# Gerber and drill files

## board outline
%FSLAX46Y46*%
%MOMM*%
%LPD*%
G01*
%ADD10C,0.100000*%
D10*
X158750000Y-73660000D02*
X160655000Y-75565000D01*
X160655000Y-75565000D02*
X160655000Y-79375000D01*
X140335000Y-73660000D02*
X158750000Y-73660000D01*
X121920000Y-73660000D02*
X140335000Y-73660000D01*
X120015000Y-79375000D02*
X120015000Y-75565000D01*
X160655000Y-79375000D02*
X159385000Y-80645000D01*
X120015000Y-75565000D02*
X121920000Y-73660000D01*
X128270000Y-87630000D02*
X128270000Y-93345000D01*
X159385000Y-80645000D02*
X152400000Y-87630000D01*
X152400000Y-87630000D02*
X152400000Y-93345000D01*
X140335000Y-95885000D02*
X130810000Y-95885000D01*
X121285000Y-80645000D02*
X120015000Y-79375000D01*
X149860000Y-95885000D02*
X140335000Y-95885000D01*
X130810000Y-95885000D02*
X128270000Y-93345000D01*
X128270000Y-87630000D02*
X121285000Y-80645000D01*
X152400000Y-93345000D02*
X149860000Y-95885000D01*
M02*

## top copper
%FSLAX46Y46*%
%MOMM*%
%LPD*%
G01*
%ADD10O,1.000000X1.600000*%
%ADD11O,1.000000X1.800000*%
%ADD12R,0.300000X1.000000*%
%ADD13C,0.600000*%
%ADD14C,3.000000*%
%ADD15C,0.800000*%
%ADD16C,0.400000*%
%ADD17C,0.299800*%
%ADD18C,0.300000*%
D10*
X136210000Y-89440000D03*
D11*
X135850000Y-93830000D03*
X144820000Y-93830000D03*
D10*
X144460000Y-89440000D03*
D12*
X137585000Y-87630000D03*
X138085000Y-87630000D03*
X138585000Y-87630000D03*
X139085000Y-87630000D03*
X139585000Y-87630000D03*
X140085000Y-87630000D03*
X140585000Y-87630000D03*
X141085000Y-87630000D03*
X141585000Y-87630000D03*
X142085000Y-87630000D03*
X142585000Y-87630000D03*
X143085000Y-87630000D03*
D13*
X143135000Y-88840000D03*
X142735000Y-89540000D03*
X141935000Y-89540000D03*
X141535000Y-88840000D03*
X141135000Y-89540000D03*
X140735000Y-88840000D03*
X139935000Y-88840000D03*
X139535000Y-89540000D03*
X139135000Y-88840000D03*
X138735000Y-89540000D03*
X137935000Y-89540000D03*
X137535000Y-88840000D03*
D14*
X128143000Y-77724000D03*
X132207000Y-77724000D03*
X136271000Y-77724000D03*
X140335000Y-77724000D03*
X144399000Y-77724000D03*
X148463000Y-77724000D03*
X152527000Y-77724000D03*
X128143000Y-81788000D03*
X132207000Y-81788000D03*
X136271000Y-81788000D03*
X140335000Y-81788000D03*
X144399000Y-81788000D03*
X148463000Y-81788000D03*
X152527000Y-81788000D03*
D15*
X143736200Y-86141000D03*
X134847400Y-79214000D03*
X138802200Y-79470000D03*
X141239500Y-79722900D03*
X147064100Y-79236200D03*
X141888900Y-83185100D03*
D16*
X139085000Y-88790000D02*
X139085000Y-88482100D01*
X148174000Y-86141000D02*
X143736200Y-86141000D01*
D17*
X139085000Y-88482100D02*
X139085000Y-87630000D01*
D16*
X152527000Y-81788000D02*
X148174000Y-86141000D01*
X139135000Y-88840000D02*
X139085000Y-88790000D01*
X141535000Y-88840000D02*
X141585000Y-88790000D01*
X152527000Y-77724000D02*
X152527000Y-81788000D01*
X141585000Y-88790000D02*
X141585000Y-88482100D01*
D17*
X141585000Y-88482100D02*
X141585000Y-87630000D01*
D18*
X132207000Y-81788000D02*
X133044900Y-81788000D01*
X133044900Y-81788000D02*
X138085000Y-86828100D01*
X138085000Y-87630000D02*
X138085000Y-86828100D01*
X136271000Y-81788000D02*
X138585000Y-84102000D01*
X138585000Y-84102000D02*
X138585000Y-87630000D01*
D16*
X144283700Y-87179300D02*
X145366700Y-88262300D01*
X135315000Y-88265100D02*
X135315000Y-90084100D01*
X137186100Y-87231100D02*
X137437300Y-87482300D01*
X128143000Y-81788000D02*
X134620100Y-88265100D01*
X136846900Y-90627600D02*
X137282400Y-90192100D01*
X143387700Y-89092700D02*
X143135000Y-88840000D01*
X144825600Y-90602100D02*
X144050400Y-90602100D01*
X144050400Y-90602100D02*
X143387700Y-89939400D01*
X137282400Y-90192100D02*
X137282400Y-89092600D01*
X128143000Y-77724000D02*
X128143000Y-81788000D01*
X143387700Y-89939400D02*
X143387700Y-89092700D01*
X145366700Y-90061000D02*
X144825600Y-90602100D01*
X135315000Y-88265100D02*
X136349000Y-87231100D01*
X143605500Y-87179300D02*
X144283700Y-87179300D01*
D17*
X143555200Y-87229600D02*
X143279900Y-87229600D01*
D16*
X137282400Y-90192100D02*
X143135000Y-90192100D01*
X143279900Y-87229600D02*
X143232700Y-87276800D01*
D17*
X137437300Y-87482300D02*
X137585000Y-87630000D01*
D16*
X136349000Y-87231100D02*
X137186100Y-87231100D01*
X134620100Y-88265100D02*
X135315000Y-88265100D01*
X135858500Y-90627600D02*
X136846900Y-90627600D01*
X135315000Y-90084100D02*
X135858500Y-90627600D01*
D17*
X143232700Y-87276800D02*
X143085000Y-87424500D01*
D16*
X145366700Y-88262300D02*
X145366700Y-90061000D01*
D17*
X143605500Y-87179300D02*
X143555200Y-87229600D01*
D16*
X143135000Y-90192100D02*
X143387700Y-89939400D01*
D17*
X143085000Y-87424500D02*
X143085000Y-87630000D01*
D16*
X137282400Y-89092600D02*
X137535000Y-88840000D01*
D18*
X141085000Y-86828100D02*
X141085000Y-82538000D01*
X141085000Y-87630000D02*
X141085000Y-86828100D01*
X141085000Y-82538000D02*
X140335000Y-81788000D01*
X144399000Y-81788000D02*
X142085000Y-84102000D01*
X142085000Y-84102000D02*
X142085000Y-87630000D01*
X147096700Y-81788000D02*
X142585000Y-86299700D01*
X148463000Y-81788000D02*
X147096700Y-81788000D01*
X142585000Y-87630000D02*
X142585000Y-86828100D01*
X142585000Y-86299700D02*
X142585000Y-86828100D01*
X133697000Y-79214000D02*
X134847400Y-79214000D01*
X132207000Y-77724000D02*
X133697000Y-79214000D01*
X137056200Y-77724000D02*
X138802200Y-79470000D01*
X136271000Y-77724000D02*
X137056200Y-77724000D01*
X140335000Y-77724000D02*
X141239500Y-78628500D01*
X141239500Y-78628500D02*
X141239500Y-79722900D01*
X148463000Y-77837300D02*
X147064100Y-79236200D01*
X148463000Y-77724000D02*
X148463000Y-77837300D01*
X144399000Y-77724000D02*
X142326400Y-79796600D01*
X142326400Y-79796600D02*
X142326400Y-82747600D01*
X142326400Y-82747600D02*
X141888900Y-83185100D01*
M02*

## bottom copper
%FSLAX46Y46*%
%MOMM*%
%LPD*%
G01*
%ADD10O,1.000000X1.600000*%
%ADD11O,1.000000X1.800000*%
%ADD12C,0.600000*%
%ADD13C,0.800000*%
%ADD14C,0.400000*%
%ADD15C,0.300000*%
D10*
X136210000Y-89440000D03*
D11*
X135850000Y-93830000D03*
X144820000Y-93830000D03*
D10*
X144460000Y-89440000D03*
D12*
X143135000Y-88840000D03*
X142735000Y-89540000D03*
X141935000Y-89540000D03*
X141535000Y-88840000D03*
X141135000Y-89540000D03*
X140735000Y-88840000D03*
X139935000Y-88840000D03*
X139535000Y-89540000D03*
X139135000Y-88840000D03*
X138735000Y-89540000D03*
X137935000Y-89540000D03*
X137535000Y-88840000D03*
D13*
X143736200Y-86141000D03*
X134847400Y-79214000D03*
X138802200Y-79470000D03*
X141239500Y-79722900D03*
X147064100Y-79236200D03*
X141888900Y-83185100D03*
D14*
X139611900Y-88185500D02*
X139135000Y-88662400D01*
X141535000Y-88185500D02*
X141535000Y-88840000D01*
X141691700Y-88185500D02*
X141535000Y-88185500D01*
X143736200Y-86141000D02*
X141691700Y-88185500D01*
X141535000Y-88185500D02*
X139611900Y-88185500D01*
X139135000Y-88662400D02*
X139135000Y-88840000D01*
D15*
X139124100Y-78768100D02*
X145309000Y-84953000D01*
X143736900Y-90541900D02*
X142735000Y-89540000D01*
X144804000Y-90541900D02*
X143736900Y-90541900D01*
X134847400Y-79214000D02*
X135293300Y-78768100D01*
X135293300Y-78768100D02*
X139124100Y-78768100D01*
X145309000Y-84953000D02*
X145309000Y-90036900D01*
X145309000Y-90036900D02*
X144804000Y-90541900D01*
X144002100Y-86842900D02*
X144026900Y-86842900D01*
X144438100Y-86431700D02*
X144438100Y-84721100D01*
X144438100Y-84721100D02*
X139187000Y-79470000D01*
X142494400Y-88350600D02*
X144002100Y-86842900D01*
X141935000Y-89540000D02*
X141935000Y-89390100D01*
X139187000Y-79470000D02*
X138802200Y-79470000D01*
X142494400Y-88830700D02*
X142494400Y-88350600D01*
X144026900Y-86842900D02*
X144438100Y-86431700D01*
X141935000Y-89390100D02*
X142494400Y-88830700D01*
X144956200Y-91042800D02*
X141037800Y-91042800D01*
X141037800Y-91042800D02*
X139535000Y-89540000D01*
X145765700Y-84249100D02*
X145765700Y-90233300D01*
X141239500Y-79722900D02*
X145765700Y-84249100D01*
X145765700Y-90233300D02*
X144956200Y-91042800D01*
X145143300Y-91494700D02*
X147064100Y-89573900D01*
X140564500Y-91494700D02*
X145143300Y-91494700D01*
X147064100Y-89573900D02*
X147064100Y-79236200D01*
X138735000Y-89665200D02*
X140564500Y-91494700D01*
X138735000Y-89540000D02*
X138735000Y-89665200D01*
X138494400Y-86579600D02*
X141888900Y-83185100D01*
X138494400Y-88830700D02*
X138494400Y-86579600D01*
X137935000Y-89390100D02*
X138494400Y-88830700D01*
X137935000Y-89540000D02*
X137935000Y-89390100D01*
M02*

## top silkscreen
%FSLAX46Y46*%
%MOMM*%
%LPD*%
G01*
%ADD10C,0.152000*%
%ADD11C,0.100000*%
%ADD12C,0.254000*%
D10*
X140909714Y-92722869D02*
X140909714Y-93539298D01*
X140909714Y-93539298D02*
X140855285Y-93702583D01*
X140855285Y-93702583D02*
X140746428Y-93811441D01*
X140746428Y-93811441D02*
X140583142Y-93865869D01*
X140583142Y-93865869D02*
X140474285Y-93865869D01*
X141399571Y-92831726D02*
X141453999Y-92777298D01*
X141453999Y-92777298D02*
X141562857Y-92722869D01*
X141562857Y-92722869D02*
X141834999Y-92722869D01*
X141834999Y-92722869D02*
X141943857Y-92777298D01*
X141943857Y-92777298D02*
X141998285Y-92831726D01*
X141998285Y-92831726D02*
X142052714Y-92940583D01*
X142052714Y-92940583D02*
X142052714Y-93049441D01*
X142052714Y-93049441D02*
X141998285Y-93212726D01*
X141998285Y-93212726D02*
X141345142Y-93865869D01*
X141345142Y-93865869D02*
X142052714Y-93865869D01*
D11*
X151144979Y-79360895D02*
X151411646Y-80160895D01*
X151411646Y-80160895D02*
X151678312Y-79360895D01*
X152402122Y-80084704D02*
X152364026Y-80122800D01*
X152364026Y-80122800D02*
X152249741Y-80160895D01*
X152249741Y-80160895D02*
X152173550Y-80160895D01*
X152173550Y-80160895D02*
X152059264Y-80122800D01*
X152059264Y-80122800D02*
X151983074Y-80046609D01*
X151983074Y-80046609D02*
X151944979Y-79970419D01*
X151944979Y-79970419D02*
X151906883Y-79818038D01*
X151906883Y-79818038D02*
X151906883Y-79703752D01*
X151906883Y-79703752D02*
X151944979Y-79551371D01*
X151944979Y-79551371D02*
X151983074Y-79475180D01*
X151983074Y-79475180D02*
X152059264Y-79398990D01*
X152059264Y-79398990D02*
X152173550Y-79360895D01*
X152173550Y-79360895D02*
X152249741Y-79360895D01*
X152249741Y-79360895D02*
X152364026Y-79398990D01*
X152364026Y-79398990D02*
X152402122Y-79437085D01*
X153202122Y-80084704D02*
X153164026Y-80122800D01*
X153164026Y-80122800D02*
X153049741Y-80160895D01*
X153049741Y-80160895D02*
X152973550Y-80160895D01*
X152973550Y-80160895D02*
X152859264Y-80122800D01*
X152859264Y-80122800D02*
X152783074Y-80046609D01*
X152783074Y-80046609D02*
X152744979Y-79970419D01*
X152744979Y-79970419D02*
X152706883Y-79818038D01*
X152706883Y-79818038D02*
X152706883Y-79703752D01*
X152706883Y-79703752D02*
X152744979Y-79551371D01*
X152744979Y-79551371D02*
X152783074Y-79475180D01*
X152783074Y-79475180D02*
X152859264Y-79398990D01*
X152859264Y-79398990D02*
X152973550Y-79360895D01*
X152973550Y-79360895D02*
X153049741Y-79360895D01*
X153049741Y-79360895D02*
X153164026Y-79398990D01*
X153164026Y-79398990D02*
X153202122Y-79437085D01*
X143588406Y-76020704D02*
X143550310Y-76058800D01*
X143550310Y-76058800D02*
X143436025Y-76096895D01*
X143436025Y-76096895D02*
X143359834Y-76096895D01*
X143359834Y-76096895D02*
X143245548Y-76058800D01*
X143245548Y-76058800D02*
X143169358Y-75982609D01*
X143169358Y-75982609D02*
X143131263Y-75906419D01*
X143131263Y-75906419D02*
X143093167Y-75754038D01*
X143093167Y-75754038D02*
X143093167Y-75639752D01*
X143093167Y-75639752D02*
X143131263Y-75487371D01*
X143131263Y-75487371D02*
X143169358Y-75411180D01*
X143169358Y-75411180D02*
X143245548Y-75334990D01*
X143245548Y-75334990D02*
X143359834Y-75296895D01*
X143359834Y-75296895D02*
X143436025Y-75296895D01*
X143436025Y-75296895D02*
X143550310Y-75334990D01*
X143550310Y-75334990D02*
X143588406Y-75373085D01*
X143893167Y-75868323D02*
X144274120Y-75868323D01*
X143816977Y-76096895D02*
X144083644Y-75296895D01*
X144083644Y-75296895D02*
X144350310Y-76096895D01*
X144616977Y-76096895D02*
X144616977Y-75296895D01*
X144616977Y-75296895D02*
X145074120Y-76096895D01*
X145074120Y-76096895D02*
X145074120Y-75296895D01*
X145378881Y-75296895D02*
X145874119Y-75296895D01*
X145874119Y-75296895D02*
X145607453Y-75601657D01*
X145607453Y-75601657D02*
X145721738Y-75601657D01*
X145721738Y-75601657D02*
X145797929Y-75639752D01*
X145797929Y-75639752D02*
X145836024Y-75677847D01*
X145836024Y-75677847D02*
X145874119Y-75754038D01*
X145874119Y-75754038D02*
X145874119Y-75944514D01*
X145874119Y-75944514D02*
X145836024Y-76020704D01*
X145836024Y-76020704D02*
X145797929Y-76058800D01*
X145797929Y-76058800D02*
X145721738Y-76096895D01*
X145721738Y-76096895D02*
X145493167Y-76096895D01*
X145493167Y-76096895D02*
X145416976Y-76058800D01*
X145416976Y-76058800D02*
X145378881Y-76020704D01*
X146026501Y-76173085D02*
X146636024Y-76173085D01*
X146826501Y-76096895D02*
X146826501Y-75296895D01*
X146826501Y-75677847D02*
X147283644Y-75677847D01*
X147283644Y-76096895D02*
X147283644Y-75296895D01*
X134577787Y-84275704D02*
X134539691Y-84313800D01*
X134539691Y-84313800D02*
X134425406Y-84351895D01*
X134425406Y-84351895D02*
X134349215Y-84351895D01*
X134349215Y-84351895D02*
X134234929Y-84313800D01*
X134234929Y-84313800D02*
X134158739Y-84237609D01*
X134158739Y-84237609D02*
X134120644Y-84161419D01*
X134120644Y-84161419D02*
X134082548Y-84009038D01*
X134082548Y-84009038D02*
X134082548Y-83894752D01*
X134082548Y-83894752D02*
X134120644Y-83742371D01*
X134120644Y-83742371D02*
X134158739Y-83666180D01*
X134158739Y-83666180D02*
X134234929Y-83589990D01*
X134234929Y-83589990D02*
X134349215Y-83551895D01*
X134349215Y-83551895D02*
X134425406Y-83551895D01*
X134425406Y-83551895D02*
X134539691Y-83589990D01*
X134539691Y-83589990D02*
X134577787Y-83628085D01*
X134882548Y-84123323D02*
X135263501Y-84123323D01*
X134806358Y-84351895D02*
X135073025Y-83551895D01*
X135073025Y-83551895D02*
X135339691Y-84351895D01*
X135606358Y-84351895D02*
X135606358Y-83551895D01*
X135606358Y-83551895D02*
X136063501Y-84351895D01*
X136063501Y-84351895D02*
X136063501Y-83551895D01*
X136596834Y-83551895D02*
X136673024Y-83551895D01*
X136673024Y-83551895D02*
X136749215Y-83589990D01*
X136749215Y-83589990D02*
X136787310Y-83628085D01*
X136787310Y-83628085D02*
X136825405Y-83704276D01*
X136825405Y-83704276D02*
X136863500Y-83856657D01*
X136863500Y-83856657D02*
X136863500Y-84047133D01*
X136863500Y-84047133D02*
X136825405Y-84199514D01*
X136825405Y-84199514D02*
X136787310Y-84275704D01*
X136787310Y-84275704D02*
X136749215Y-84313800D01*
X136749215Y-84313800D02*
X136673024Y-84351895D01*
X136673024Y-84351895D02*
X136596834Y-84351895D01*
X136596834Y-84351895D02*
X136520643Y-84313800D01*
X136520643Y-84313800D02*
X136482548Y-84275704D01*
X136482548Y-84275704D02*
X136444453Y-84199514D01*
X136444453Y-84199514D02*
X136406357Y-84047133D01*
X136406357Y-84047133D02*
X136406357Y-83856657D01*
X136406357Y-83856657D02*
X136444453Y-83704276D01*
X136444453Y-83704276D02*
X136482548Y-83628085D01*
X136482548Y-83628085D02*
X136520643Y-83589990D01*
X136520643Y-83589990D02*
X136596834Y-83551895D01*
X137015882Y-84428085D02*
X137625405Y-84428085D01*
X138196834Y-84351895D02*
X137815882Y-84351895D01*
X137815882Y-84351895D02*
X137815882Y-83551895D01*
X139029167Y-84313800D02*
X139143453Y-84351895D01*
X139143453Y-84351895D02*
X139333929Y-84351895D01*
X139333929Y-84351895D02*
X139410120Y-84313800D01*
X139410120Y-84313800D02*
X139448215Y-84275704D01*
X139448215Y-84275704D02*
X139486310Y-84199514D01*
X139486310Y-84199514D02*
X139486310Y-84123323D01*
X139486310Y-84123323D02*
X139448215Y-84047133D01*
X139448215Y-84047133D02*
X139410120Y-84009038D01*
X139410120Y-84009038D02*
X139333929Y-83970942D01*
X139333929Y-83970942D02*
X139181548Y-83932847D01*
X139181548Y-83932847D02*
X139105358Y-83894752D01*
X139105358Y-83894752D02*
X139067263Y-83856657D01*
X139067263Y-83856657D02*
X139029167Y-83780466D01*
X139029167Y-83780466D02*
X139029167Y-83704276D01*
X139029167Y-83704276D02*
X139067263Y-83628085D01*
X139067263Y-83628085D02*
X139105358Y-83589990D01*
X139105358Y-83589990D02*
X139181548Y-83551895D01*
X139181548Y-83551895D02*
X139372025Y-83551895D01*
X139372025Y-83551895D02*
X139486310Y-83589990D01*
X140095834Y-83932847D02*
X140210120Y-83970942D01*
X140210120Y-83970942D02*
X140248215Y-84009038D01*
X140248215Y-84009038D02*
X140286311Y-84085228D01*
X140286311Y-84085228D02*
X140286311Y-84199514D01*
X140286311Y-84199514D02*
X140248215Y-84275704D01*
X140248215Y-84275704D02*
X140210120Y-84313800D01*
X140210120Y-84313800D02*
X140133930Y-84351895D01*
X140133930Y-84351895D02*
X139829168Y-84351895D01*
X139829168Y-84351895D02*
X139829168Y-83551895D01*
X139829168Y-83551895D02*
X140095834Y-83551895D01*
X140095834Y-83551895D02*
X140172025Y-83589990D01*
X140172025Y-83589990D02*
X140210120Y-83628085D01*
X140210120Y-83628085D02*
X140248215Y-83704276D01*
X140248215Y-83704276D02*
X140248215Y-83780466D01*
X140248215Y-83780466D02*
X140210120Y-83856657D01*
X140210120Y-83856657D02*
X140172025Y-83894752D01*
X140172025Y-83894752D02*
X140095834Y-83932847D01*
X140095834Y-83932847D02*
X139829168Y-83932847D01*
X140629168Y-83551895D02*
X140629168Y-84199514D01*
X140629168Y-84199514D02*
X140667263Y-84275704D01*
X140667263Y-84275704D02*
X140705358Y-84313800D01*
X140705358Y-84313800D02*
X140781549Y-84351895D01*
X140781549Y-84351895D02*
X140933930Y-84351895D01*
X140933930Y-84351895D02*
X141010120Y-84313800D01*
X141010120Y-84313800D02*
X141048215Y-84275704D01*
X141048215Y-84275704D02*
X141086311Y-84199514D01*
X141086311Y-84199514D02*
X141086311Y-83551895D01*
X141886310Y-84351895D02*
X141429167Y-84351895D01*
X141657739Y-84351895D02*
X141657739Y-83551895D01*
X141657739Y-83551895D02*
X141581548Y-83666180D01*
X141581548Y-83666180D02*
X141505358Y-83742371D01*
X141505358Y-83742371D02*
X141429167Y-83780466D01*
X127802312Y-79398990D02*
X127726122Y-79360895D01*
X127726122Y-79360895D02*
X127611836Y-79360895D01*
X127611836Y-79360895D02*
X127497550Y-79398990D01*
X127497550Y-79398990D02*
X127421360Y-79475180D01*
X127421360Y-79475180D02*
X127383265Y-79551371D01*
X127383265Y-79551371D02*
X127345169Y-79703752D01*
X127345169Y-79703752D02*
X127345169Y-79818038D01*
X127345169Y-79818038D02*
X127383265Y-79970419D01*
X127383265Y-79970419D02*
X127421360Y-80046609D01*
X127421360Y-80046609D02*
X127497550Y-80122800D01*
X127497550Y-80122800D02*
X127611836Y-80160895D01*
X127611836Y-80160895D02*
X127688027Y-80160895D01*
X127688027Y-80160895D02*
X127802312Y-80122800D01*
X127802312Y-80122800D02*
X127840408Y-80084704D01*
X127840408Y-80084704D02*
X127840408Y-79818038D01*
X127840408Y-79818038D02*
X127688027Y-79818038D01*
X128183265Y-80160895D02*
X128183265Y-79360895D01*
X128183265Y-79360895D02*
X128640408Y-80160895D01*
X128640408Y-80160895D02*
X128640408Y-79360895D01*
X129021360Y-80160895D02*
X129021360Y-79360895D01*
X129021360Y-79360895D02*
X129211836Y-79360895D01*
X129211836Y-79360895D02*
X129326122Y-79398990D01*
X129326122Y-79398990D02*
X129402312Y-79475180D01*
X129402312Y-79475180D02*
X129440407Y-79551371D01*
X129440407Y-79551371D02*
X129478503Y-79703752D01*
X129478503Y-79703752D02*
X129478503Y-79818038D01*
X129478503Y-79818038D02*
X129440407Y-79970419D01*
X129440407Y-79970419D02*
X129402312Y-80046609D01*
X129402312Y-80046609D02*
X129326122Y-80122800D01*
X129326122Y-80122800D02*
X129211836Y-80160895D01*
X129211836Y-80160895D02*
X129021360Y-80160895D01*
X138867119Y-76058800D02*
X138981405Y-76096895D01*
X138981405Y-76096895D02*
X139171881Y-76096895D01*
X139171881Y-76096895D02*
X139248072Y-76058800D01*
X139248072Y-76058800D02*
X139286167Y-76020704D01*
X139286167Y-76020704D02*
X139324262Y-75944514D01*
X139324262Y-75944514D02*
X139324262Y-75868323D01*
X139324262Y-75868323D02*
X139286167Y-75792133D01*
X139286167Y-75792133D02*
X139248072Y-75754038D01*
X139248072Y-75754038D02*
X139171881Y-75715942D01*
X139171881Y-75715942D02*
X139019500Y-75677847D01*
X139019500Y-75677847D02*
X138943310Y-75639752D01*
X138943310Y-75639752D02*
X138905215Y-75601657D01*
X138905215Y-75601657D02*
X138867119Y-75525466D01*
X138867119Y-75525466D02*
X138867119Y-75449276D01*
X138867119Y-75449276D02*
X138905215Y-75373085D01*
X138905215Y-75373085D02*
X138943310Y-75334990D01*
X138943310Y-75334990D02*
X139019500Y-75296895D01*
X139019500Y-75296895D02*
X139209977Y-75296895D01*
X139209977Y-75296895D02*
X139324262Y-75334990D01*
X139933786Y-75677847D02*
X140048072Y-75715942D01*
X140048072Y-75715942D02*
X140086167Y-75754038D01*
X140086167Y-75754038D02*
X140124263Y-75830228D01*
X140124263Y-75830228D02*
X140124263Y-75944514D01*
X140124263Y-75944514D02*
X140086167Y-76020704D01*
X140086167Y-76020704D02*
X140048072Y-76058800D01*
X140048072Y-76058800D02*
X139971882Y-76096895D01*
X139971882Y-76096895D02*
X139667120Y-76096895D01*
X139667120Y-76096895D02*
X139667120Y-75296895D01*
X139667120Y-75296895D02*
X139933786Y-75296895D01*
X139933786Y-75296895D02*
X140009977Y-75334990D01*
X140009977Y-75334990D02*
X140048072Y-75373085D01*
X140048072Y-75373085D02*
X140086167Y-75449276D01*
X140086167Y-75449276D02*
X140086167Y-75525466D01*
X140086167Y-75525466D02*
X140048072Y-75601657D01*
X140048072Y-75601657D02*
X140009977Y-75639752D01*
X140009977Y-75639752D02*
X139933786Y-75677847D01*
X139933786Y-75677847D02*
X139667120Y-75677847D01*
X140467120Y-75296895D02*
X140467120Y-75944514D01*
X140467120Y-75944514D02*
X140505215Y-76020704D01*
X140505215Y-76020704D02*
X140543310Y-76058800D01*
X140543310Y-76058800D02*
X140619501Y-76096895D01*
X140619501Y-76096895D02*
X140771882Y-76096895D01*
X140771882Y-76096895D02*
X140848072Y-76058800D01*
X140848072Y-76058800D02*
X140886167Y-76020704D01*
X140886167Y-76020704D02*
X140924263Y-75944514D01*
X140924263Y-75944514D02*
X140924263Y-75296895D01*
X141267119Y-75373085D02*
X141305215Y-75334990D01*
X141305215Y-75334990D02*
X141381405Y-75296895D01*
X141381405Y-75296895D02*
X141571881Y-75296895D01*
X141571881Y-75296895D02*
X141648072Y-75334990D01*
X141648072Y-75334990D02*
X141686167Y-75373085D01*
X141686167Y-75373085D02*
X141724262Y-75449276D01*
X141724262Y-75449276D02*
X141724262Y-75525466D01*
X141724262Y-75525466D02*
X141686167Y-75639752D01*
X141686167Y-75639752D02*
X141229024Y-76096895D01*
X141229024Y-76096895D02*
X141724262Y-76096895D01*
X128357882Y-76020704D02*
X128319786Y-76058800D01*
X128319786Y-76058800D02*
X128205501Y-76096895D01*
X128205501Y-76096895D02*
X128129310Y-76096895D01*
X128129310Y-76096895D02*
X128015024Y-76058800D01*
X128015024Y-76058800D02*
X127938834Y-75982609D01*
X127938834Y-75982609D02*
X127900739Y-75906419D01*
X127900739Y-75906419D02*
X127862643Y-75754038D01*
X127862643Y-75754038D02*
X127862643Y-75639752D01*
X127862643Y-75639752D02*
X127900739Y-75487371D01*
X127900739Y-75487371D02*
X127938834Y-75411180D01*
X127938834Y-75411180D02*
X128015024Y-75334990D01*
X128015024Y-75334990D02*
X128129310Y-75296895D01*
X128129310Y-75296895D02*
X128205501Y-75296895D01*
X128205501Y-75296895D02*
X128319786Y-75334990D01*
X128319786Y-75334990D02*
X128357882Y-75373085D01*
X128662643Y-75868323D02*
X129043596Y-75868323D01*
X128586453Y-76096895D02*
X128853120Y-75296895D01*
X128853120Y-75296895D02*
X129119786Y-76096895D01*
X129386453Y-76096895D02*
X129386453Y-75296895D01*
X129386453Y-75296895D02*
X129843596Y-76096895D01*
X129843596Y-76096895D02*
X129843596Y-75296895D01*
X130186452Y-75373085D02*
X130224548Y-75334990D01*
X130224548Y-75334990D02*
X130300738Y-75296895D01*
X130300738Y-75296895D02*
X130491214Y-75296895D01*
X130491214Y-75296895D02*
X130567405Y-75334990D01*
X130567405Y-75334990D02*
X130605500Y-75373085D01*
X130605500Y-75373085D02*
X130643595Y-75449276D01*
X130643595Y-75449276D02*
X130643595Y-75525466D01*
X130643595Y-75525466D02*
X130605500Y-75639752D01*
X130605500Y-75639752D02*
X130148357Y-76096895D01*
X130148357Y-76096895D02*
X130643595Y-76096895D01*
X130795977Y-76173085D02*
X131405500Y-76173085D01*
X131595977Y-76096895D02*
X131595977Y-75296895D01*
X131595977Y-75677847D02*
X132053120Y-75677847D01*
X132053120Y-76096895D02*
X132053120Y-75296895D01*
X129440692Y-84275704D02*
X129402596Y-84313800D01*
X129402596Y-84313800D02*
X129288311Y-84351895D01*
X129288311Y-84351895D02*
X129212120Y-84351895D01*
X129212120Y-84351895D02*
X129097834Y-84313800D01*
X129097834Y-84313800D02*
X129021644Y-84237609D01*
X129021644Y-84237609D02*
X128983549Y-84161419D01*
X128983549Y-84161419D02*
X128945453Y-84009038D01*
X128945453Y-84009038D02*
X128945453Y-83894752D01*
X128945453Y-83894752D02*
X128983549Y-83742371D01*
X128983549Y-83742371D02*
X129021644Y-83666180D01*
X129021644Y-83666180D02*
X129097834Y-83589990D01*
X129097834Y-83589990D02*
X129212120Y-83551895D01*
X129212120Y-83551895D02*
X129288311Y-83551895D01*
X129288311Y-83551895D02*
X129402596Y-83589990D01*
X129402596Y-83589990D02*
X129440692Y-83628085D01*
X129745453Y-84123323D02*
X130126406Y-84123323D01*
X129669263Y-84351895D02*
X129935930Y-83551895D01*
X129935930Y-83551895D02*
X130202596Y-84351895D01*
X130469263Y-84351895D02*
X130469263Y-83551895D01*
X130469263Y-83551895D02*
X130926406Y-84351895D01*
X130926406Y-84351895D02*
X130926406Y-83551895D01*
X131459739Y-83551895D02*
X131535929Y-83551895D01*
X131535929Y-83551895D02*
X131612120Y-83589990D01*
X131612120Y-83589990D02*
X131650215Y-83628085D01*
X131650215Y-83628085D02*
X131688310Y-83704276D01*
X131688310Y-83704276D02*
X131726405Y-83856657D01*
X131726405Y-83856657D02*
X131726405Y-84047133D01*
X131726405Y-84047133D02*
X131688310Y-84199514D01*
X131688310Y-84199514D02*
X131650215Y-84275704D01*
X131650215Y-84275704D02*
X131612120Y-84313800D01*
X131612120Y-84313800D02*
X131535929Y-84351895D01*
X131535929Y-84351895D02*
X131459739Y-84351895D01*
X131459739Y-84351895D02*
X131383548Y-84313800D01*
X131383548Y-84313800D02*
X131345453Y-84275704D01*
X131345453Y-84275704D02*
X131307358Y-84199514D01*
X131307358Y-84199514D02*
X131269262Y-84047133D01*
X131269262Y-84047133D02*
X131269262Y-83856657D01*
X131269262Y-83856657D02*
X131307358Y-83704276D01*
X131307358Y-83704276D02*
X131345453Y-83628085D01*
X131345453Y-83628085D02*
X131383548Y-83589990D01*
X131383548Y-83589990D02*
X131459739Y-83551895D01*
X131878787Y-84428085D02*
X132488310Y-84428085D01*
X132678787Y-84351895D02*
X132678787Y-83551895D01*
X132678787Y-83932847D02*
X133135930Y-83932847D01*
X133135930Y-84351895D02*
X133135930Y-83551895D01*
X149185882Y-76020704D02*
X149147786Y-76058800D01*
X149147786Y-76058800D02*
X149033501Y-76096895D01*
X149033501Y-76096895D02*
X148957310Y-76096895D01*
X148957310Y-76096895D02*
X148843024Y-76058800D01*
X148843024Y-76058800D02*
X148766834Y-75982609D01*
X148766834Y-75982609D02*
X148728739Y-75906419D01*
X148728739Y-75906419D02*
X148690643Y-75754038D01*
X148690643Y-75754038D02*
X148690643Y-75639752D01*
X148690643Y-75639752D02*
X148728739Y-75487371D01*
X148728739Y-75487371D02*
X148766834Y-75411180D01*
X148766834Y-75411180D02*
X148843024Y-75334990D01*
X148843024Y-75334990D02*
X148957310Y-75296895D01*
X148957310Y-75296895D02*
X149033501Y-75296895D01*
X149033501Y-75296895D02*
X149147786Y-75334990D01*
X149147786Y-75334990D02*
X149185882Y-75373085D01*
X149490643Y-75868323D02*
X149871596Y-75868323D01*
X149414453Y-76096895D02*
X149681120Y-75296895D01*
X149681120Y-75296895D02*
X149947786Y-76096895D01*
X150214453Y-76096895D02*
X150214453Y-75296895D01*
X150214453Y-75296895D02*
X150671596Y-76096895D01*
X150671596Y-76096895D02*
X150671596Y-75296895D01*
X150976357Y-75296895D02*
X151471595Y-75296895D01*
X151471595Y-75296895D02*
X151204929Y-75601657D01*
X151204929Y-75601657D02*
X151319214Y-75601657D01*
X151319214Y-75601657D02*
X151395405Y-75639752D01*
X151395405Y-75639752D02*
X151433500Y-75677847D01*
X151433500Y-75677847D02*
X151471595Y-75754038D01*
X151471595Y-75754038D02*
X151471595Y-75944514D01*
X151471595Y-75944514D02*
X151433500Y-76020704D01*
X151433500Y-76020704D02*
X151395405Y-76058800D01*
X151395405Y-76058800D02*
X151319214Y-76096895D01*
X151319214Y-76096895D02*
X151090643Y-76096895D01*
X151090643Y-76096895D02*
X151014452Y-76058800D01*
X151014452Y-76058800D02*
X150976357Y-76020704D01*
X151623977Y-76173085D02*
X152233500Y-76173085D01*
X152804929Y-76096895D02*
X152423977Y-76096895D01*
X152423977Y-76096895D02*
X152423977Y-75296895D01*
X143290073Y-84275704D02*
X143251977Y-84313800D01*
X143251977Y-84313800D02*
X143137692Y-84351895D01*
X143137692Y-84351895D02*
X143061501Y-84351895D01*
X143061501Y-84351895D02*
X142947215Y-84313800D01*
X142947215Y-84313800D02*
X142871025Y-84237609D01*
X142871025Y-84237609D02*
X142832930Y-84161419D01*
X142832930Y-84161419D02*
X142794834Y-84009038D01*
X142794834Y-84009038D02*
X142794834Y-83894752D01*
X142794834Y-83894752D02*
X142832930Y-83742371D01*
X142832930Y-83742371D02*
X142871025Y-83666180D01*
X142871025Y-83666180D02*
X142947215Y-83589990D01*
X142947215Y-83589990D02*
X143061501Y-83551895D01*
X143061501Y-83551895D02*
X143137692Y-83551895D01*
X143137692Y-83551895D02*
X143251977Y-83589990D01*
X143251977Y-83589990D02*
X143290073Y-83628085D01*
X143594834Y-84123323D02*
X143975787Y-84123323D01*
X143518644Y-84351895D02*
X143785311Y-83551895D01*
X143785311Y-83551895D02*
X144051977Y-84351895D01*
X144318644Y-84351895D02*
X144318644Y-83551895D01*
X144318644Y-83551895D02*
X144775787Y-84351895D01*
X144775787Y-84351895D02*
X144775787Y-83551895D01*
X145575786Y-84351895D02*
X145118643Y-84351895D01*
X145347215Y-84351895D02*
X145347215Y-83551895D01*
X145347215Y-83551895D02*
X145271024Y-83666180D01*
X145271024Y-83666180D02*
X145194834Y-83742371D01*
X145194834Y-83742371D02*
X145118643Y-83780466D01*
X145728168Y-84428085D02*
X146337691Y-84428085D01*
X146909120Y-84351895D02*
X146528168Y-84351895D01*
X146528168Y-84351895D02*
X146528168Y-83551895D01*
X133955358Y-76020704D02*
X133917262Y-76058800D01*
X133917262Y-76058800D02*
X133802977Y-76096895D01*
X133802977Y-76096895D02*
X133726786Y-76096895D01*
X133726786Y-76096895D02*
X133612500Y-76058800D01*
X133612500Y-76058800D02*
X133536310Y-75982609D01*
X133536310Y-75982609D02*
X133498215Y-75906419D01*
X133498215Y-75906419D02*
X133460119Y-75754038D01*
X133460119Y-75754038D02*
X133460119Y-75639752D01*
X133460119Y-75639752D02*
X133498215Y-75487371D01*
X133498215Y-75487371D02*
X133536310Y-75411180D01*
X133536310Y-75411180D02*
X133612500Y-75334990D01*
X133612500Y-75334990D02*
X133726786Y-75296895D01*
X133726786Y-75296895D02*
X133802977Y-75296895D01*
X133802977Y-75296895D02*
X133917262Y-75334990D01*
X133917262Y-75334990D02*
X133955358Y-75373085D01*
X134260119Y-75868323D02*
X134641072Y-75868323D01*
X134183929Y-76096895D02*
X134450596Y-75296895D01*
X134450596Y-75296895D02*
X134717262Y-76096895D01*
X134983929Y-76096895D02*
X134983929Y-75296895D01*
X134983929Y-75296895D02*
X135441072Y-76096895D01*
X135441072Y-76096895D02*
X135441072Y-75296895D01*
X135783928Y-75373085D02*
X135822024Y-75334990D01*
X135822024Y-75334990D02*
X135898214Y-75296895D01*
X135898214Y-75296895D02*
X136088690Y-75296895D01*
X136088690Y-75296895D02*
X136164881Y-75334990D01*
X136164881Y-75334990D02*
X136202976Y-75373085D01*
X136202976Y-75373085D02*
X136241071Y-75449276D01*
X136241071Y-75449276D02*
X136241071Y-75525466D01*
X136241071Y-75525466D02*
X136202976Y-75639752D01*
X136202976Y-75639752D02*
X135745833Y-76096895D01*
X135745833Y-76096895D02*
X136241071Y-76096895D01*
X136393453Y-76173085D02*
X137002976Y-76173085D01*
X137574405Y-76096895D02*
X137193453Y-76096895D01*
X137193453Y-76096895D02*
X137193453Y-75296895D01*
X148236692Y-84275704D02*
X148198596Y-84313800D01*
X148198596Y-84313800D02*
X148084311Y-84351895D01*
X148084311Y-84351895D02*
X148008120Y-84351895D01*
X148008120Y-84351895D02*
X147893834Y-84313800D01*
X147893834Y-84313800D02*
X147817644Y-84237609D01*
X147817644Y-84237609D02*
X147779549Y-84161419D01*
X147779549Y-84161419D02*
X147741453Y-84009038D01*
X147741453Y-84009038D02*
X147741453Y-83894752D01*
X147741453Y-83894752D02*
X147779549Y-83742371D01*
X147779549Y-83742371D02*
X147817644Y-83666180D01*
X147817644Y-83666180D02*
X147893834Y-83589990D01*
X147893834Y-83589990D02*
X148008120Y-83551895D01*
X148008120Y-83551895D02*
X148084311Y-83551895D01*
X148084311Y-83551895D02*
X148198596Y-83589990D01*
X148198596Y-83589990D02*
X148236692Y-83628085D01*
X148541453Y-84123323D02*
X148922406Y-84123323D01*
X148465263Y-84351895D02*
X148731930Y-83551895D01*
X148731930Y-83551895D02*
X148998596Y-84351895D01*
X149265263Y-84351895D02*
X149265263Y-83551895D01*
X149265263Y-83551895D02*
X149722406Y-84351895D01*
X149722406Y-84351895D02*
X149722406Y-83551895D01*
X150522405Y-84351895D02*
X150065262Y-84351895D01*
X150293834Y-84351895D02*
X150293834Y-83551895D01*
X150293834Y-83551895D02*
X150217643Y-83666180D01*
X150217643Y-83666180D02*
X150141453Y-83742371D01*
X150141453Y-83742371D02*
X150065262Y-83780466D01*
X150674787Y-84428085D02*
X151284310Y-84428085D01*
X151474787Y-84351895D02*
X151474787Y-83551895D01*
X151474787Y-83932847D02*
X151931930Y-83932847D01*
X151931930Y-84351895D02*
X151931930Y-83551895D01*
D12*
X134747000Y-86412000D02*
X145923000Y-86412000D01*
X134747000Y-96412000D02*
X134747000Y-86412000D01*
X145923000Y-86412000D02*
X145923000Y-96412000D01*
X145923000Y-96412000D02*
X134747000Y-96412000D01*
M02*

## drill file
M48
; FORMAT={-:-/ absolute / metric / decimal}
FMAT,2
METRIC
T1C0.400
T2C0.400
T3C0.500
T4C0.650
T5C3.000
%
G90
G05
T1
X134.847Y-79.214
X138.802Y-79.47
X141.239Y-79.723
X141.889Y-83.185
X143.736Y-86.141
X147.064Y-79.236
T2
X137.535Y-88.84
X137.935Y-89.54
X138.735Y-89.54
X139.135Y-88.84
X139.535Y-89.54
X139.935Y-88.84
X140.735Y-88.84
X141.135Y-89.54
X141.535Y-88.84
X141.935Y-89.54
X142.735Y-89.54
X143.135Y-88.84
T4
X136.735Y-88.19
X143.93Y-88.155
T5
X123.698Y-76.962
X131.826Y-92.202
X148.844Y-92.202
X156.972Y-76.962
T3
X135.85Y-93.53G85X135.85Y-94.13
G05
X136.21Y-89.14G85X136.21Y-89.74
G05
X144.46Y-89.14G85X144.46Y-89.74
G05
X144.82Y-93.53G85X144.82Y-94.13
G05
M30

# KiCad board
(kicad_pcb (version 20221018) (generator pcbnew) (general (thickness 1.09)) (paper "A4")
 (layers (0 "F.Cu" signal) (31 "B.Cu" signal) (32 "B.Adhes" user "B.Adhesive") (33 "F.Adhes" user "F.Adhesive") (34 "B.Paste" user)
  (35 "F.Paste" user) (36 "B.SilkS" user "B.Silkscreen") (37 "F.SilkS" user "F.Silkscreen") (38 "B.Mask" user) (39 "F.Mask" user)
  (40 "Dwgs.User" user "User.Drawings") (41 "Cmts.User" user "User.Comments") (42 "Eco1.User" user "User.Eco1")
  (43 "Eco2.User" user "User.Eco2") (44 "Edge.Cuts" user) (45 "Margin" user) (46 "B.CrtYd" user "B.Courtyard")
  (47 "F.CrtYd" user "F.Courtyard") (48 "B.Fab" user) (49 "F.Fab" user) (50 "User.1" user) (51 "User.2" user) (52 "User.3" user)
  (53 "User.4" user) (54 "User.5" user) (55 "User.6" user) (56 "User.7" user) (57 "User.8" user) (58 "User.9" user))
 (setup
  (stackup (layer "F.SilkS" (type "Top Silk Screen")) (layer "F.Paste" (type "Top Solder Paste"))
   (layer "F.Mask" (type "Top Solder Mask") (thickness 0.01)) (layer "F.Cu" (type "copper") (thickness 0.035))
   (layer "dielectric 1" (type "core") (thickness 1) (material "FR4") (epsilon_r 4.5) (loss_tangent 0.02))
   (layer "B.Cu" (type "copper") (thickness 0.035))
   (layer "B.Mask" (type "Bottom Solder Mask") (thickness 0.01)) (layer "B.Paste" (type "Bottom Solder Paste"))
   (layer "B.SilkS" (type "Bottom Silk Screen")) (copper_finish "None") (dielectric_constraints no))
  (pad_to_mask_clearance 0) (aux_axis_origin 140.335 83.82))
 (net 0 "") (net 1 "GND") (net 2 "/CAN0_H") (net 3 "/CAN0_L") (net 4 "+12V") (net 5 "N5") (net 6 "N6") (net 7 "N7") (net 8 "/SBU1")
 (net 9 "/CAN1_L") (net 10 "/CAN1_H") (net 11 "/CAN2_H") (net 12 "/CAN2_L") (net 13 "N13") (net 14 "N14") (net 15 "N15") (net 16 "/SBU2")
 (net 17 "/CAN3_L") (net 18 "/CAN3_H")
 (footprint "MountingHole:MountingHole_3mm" (layer "F.Cu") (at 123.698 76.962)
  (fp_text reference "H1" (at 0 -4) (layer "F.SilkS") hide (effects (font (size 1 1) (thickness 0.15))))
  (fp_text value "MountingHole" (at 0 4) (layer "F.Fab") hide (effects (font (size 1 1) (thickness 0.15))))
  (pad "" np_thru_hole circle (at 0 0) (size 3 3) (drill 3) (layers "*.Cu" "*.Mask")))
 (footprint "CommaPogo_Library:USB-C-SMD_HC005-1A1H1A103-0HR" (layer "F.Cu") (at 140.335 90.73)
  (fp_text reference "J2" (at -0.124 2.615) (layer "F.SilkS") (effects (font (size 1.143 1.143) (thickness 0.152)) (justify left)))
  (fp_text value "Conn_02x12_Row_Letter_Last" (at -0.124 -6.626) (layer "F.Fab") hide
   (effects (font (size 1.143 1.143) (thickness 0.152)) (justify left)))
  (fp_line (start -5.588 -4.318) (end 5.588 -4.318) (stroke (width 0.254) (type solid)) (layer "F.SilkS"))
  (fp_line (start -5.588 5.682) (end -5.588 -4.318) (stroke (width 0.254) (type solid)) (layer "F.SilkS"))
  (fp_line (start 5.588 -4.318) (end 5.588 5.682) (stroke (width 0.254) (type solid)) (layer "F.SilkS"))
  (fp_line (start 5.588 5.682) (end -5.588 5.682) (stroke (width 0.254) (type solid)) (layer "F.SilkS"))
  (pad "" np_thru_hole circle (at -3.6 -2.54) (size 0.65 0.65) (drill 0.65) (layers "*.Cu" "*.Mask"))
  (pad "" np_thru_hole circle (at 3.595 -2.575) (size 0.65 0.65) (drill 0.65) (layers "*.Cu" "*.Mask"))
  (pad "1" thru_hole oval (at -4.125 -1.29) (size 1 1.6) (drill oval 0.5 1.1) (layers "*.Cu" "*.Paste" "*.Mask"))
  (pad "2" thru_hole oval (at -4.485 3.1) (size 1 1.8) (drill oval 0.5 1.1) (layers "*.Cu" "*.Paste" "*.Mask"))
  (pad "3" thru_hole oval (at 4.485 3.1) (size 1 1.8) (drill oval 0.5 1.1) (layers "*.Cu" "*.Paste" "*.Mask"))
  (pad "4" thru_hole oval (at 4.125 -1.29) (size 1 1.6) (drill oval 0.5 1.1) (layers "*.Cu" "*.Paste" "*.Mask"))
  (pad "A1" smd rect (at -2.75 -3.1) (size 0.3 1) (layers "F.Cu" "F.Paste" "F.Mask") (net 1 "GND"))
  (pad "A2" smd rect (at -2.25 -3.1) (size 0.3 1) (layers "F.Cu" "F.Paste" "F.Mask") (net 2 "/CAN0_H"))
  (pad "A3" smd rect (at -1.75 -3.1) (size 0.3 1) (layers "F.Cu" "F.Paste" "F.Mask") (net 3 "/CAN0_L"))
  (pad "A4" smd rect (at -1.25 -3.1) (size 0.3 1) (layers "F.Cu" "F.Paste" "F.Mask") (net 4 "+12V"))
  (pad "A5" smd rect (at -0.75 -3.1) (size 0.3 1) (layers "F.Cu" "F.Paste" "F.Mask") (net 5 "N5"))
  (pad "A6" smd rect (at -0.25 -3.1) (size 0.3 1) (layers "F.Cu" "F.Paste" "F.Mask") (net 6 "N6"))
  (pad "A7" smd rect (at 0.25 -3.1) (size 0.3 1) (layers "F.Cu" "F.Paste" "F.Mask") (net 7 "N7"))
  (pad "A8" smd rect (at 0.75 -3.1) (size 0.3 1) (layers "F.Cu" "F.Paste" "F.Mask") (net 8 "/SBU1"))
  (pad "A9" smd rect (at 1.25 -3.1) (size 0.3 1) (layers "F.Cu" "F.Paste" "F.Mask") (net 4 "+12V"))
  (pad "A10" smd rect (at 1.75 -3.1) (size 0.3 1) (layers "F.Cu" "F.Paste" "F.Mask") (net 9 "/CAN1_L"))
  (pad "A11" smd rect (at 2.25 -3.1) (size 0.3 1) (layers "F.Cu" "F.Paste" "F.Mask") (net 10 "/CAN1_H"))
  (pad "A12" smd rect (at 2.75 -3.1) (size 0.3 1) (layers "F.Cu" "F.Paste" "F.Mask") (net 1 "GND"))
  (pad "B1" thru_hole circle (at 2.8 -1.89) (size 0.6 0.6) (drill 0.4) (layers "*.Cu" "*.Paste" "*.Mask") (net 1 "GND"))
  (pad "B2" thru_hole circle (at 2.4 -1.19) (size 0.6 0.6) (drill 0.4) (layers "*.Cu" "*.Paste" "*.Mask") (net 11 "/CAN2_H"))
  (pad "B3" thru_hole circle (at 1.6 -1.19) (size 0.6 0.6) (drill 0.4) (layers "*.Cu" "*.Paste" "*.Mask") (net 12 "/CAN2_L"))
  (pad "B4" thru_hole circle (at 1.2 -1.89) (size 0.6 0.6) (drill 0.4) (layers "*.Cu" "*.Paste" "*.Mask") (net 4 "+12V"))
  (pad "B5" thru_hole circle (at 0.8 -1.19) (size 0.6 0.6) (drill 0.4) (layers "*.Cu" "*.Paste" "*.Mask") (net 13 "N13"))
  (pad "B6" thru_hole circle (at 0.4 -1.89) (size 0.6 0.6) (drill 0.4) (layers "*.Cu" "*.Paste" "*.Mask") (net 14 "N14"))
  (pad "B7" thru_hole circle (at -0.4 -1.89) (size 0.6 0.6) (drill 0.4) (layers "*.Cu" "*.Paste" "*.Mask") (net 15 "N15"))
  (pad "B8" thru_hole circle (at -0.8 -1.19) (size 0.6 0.6) (drill 0.4) (layers "*.Cu" "*.Paste" "*.Mask") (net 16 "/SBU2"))
  (pad "B9" thru_hole circle (at -1.2 -1.89) (size 0.6 0.6) (drill 0.4) (layers "*.Cu" "*.Paste" "*.Mask") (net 4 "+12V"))
  (pad "B10" thru_hole circle (at -1.6 -1.19) (size 0.6 0.6) (drill 0.4) (layers "*.Cu" "*.Paste" "*.Mask") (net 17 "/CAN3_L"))
  (pad "B11" thru_hole circle (at -2.4 -1.19) (size 0.6 0.6) (drill 0.4) (layers "*.Cu" "*.Paste" "*.Mask") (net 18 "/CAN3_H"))
  (pad "B12" thru_hole circle (at -2.8 -1.89) (size 0.6 0.6) (drill 0.4) (layers "*.Cu" "*.Paste" "*.Mask") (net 1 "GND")))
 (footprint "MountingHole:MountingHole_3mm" (layer "F.Cu") (at 148.844 92.202)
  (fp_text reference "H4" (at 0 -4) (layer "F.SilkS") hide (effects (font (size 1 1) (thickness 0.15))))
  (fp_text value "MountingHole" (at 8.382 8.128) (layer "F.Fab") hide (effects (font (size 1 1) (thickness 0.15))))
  (pad "" np_thru_hole circle (at 0 0) (size 3 3) (drill 3) (layers "*.Cu" "*.Mask")))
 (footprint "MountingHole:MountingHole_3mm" (layer "F.Cu") (at 131.826 92.202)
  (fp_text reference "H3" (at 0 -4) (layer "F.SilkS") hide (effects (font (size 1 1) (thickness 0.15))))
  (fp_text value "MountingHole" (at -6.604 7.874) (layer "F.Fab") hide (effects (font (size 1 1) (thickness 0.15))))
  (pad "" np_thru_hole circle (at 0 0) (size 3 3) (drill 3) (layers "*.Cu" "*.Mask")))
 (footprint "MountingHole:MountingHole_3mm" (layer "F.Cu") (at 156.972 76.962)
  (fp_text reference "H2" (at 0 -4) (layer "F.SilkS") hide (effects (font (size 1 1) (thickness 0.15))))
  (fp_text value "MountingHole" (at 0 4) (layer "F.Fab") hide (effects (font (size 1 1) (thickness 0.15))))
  (pad "" np_thru_hole circle (at 0 0) (size 3 3) (drill 3) (layers "*.Cu" "*.Mask")))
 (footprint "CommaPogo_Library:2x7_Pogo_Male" (layer "F.Cu") (at 140.335 83.82)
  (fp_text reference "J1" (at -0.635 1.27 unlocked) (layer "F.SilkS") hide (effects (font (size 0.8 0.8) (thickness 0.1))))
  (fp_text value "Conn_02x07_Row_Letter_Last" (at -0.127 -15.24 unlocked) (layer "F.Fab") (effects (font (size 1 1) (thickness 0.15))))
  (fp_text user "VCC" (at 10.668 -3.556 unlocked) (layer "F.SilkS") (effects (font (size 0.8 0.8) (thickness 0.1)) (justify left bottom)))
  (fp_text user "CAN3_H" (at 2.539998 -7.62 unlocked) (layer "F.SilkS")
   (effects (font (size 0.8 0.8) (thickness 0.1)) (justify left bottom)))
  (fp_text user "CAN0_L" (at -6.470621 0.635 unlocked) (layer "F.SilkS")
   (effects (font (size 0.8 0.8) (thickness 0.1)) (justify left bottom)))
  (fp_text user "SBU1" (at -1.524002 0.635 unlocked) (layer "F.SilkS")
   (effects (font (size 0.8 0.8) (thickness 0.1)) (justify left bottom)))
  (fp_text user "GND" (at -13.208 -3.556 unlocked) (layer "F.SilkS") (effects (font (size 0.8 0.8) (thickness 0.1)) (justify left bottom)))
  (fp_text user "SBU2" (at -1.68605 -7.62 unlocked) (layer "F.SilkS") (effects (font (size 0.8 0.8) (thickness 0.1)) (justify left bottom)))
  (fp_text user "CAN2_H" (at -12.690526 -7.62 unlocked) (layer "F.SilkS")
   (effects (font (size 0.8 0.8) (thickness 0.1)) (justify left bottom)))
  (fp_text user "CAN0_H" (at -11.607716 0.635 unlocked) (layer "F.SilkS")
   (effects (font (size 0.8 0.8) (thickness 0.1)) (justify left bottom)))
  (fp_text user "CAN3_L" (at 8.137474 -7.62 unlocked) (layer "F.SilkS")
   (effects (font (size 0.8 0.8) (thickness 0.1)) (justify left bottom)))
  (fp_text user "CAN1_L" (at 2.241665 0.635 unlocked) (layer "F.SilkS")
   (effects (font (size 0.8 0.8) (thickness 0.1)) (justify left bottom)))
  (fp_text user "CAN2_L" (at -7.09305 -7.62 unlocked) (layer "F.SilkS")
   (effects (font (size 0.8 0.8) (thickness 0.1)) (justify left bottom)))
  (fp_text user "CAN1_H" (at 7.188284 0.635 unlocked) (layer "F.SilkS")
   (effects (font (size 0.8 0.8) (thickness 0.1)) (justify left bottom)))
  (pad "1" smd circle (at -12.192 -6.096) (size 3 3) (layers "F.Cu" "F.Paste" "F.Mask") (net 1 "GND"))
  (pad "2" smd circle (at -8.128 -6.096) (size 3 3) (layers "F.Cu" "F.Paste" "F.Mask") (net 11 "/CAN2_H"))
  (pad "3" smd circle (at -4.064 -6.096) (size 3 3) (layers "F.Cu" "F.Paste" "F.Mask") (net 12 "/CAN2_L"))
  (pad "4" smd circle (at 0 -6.096) (size 3 3) (layers "F.Cu" "F.Paste" "F.Mask") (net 16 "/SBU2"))
  (pad "5" smd circle (at 4.064 -6.096) (size 3 3) (layers "F.Cu" "F.Paste" "F.Mask") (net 18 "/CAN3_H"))
  (pad "6" smd circle (at 8.128 -6.096) (size 3 3) (layers "F.Cu" "F.Paste" "F.Mask") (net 17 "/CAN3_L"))
  (pad "7" smd circle (at 12.192 -6.096) (size 3 3) (layers "F.Cu" "F.Paste" "F.Mask") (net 4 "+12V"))
  (pad "8" smd circle (at -12.192 -2.032) (size 3 3) (layers "F.Cu" "F.Paste" "F.Mask") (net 1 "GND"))
  (pad "9" smd circle (at -8.128 -2.032) (size 3 3) (layers "F.Cu" "F.Paste" "F.Mask") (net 2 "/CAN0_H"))
  (pad "10" smd circle (at -4.064 -2.032) (size 3 3) (layers "F.Cu" "F.Paste" "F.Mask") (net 3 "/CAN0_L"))
  (pad "11" smd circle (at 0 -2.032) (size 3 3) (layers "F.Cu" "F.Paste" "F.Mask") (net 8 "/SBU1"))
  (pad "12" smd circle (at 4.064 -2.032) (size 3 3) (layers "F.Cu" "F.Paste" "F.Mask") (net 9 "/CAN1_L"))
  (pad "13" smd circle (at 8.128 -2.032) (size 3 3) (layers "F.Cu" "F.Paste" "F.Mask") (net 10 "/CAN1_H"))
  (pad "14" smd circle (at 12.192 -2.032) (size 3 3) (layers "F.Cu" "F.Paste" "F.Mask") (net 4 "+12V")))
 (gr_line (start 158.75 73.66) (end 160.655 75.565) (stroke (width 0.1) (type default)) (layer "Edge.Cuts"))
 (gr_line (start 160.655 75.565) (end 160.655 79.375) (stroke (width 0.1) (type default)) (layer "Edge.Cuts"))
 (gr_line (start 140.335 73.66) (end 158.75 73.66) (stroke (width 0.1) (type default)) (layer "Edge.Cuts"))
 (gr_line (start 121.92 73.66) (end 140.335 73.66) (stroke (width 0.1) (type default)) (layer "Edge.Cuts"))
 (gr_line (start 120.015 79.375) (end 120.015 75.565) (stroke (width 0.1) (type default)) (layer "Edge.Cuts"))
 (gr_line (start 160.655 79.375) (end 159.385 80.645) (stroke (width 0.1) (type default)) (layer "Edge.Cuts"))
 (gr_line (start 120.015 75.565) (end 121.92 73.66) (stroke (width 0.1) (type default)) (layer "Edge.Cuts"))
 (gr_line (start 128.27 87.63) (end 128.27 93.345) (stroke (width 0.1) (type default)) (layer "Edge.Cuts"))
 (gr_line (start 159.385 80.645) (end 152.4 87.63) (stroke (width 0.1) (type default)) (layer "Edge.Cuts"))
 (gr_line (start 152.4 87.63) (end 152.4 93.345) (stroke (width 0.1) (type default)) (layer "Edge.Cuts"))
 (gr_line (start 140.335 95.885) (end 130.81 95.885) (stroke (width 0.1) (type default)) (layer "Edge.Cuts"))
 (gr_line (start 121.285 80.645) (end 120.015 79.375) (stroke (width 0.1) (type default)) (layer "Edge.Cuts"))
 (gr_line (start 149.86 95.885) (end 140.335 95.885) (stroke (width 0.1) (type default)) (layer "Edge.Cuts"))
 (gr_line (start 130.81 95.885) (end 128.27 93.345) (stroke (width 0.1) (type default)) (layer "Edge.Cuts"))
 (gr_line (start 128.27 87.63) (end 121.285 80.645) (stroke (width 0.1) (type default)) (layer "Edge.Cuts"))
 (gr_line (start 152.4 93.345) (end 149.86 95.885) (stroke (width 0.1) (type default)) (layer "Edge.Cuts"))
 (segment (start 139.085 88.79) (end 139.085 88.4821) (width 0.4) (layer "F.Cu") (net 4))
 (segment (start 148.174 86.141) (end 143.7362 86.141) (width 0.4) (layer "F.Cu") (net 4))
 (segment (start 139.085 88.4821) (end 139.085 87.63) (width 0.2998) (layer "F.Cu") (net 4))
 (segment (start 152.527 81.788) (end 148.174 86.141) (width 0.4) (layer "F.Cu") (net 4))
 (segment (start 139.135 88.84) (end 139.085 88.79) (width 0.4) (layer "F.Cu") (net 4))
 (segment (start 141.535 88.84) (end 141.585 88.79) (width 0.4) (layer "F.Cu") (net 4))
 (segment (start 152.527 77.724) (end 152.527 81.788) (width 0.4) (layer "F.Cu") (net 4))
 (segment (start 141.585 88.79) (end 141.585 88.4821) (width 0.4) (layer "F.Cu") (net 4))
 (segment (start 141.585 88.4821) (end 141.585 87.63) (width 0.2998) (layer "F.Cu") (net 4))
 (via (at 143.7362 86.141) (size 0.8) (drill 0.4) (layers "F.Cu" "B.Cu") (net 4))
 (segment (start 139.6119 88.1855) (end 139.135 88.6624) (width 0.4) (layer "B.Cu") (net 4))
 (segment (start 141.535 88.1855) (end 141.535 88.84) (width 0.4) (layer "B.Cu") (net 4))
 (segment (start 141.6917 88.1855) (end 141.535 88.1855) (width 0.4) (layer "B.Cu") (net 4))
 (segment (start 143.7362 86.141) (end 141.6917 88.1855) (width 0.4) (layer "B.Cu") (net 4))
 (segment (start 141.535 88.1855) (end 139.6119 88.1855) (width 0.4) (layer "B.Cu") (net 4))
 (segment (start 139.135 88.6624) (end 139.135 88.84) (width 0.4) (layer "B.Cu") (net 4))
 (segment (start 132.207 81.788) (end 133.0449 81.788) (width 0.3) (layer "F.Cu") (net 2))
 (segment (start 133.0449 81.788) (end 138.085 86.8281) (width 0.3) (layer "F.Cu") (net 2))
 (segment (start 138.085 87.63) (end 138.085 86.8281) (width 0.3) (layer "F.Cu") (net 2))
 (segment (start 136.271 81.788) (end 138.585 84.102) (width 0.3) (layer "F.Cu") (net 3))
 (segment (start 138.585 84.102) (end 138.585 87.63) (width 0.3) (layer "F.Cu") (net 3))
 (segment (start 144.2837 87.1793) (end 145.3667 88.2623) (width 0.4) (layer "F.Cu") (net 1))
 (segment (start 135.315 88.2651) (end 135.315 90.0841) (width 0.4) (layer "F.Cu") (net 1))
 (segment (start 137.1861 87.2311) (end 137.4373 87.4823) (width 0.4) (layer "F.Cu") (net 1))
 (segment (start 128.143 81.788) (end 134.6201 88.2651) (width 0.4) (layer "F.Cu") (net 1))
 (segment (start 136.8469 90.6276) (end 137.2824 90.1921) (width 0.4) (layer "F.Cu") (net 1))
 (segment (start 143.3877 89.0927) (end 143.135 88.84) (width 0.4) (layer "F.Cu") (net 1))
 (segment (start 144.8256 90.6021) (end 144.0504 90.6021) (width 0.4) (layer "F.Cu") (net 1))
 (segment (start 144.0504 90.6021) (end 143.3877 89.9394) (width 0.4) (layer "F.Cu") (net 1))
 (segment (start 137.2824 90.1921) (end 137.2824 89.0926) (width 0.4) (layer "F.Cu") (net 1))
 (segment (start 128.143 77.724) (end 128.143 81.788) (width 0.4) (layer "F.Cu") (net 1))
 (segment (start 143.3877 89.9394) (end 143.3877 89.0927) (width 0.4) (layer "F.Cu") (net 1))
 (segment (start 145.3667 90.061) (end 144.8256 90.6021) (width 0.4) (layer "F.Cu") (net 1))
 (segment (start 135.315 88.2651) (end 136.349 87.2311) (width 0.4) (layer "F.Cu") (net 1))
 (segment (start 143.6055 87.1793) (end 144.2837 87.1793) (width 0.4) (layer "F.Cu") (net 1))
 (segment (start 143.5552 87.2296) (end 143.2799 87.2296) (width 0.2998) (layer "F.Cu") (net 1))
 (segment (start 137.2824 90.1921) (end 143.135 90.1921) (width 0.4) (layer "F.Cu") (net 1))
 (segment (start 143.2799 87.2296) (end 143.2327 87.2768) (width 0.4) (layer "F.Cu") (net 1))
 (segment (start 137.4373 87.4823) (end 137.585 87.63) (width 0.2998) (layer "F.Cu") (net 1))
 (segment (start 136.349 87.2311) (end 137.1861 87.2311) (width 0.4) (layer "F.Cu") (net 1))
 (segment (start 134.6201 88.2651) (end 135.315 88.2651) (width 0.4) (layer "F.Cu") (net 1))
 (segment (start 135.8585 90.6276) (end 136.8469 90.6276) (width 0.4) (layer "F.Cu") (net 1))
 (segment (start 135.315 90.0841) (end 135.8585 90.6276) (width 0.4) (layer "F.Cu") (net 1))
 (segment (start 143.2327 87.2768) (end 143.085 87.4245) (width 0.2998) (layer "F.Cu") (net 1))
 (segment (start 145.3667 88.2623) (end 145.3667 90.061) (width 0.4) (layer "F.Cu") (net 1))
 (segment (start 143.6055 87.1793) (end 143.5552 87.2296) (width 0.2998) (layer "F.Cu") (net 1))
 (segment (start 143.135 90.1921) (end 143.3877 89.9394) (width 0.4) (layer "F.Cu") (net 1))
 (segment (start 143.085 87.4245) (end 143.085 87.63) (width 0.2998) (layer "F.Cu") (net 1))
 (segment (start 137.2824 89.0926) (end 137.535 88.84) (width 0.4) (layer "F.Cu") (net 1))
 (segment (start 141.085 86.8281) (end 141.085 82.538) (width 0.3) (layer "F.Cu") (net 8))
 (segment (start 141.085 87.63) (end 141.085 86.8281) (width 0.3) (layer "F.Cu") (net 8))
 (segment (start 141.085 82.538) (end 140.335 81.788) (width 0.3) (layer "F.Cu") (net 8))
 (segment (start 144.399 81.788) (end 142.085 84.102) (width 0.3) (layer "F.Cu") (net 9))
 (segment (start 142.085 84.102) (end 142.085 87.63) (width 0.3) (layer "F.Cu") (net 9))
 (segment (start 147.0967 81.788) (end 142.585 86.2997) (width 0.3) (layer "F.Cu") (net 10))
 (segment (start 148.463 81.788) (end 147.0967 81.788) (width 0.3) (layer "F.Cu") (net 10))
 (segment (start 142.585 87.63) (end 142.585 86.8281) (width 0.3) (layer "F.Cu") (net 10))
 (segment (start 142.585 86.2997) (end 142.585 86.8281) (width 0.3) (layer "F.Cu") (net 10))
 (segment (start 133.697 79.214) (end 134.8474 79.214) (width 0.3) (layer "F.Cu") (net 11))
 (segment (start 132.207 77.724) (end 133.697 79.214) (width 0.3) (layer "F.Cu") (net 11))
 (via (at 134.8474 79.214) (size 0.8) (drill 0.4) (layers "F.Cu" "B.Cu") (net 11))
 (segment (start 139.1241 78.7681) (end 145.309 84.953) (width 0.3) (layer "B.Cu") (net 11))
 (segment (start 143.7369 90.5419) (end 142.735 89.54) (width 0.3) (layer "B.Cu") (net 11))
 (segment (start 144.804 90.5419) (end 143.7369 90.5419) (width 0.3) (layer "B.Cu") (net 11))
 (segment (start 134.8474 79.214) (end 135.2933 78.7681) (width 0.3) (layer "B.Cu") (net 11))
 (segment (start 135.2933 78.7681) (end 139.1241 78.7681) (width 0.3) (layer "B.Cu") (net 11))
 (segment (start 145.309 84.953) (end 145.309 90.0369) (width 0.3) (layer "B.Cu") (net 11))
 (segment (start 145.309 90.0369) (end 144.804 90.5419) (width 0.3) (layer "B.Cu") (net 11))
 (segment (start 137.0562 77.724) (end 138.8022 79.47) (width 0.3) (layer "F.Cu") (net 12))
 (segment (start 136.271 77.724) (end 137.0562 77.724) (width 0.3) (layer "F.Cu") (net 12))
 (via (at 138.8022 79.47) (size 0.8) (drill 0.4) (layers "F.Cu" "B.Cu") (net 12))
 (segment (start 144.0021 86.8429) (end 144.0269 86.8429) (width 0.3) (layer "B.Cu") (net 12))
 (segment (start 144.4381 86.4317) (end 144.4381 84.7211) (width 0.3) (layer "B.Cu") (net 12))
 (segment (start 144.4381 84.7211) (end 139.187 79.47) (width 0.3) (layer "B.Cu") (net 12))
 (segment (start 142.4944 88.3506) (end 144.0021 86.8429) (width 0.3) (layer "B.Cu") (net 12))
 (segment (start 141.935 89.54) (end 141.935 89.3901) (width 0.3) (layer "B.Cu") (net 12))
 (segment (start 139.187 79.47) (end 138.8022 79.47) (width 0.3) (layer "B.Cu") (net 12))
 (segment (start 142.4944 88.8307) (end 142.4944 88.3506) (width 0.3) (layer "B.Cu") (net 12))
 (segment (start 144.0269 86.8429) (end 144.4381 86.4317) (width 0.3) (layer "B.Cu") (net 12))
 (segment (start 141.935 89.3901) (end 142.4944 88.8307) (width 0.3) (layer "B.Cu") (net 12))
 (segment (start 140.335 77.724) (end 141.2395 78.6285) (width 0.3) (layer "F.Cu") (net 16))
 (segment (start 141.2395 78.6285) (end 141.2395 79.7229) (width 0.3) (layer "F.Cu") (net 16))
 (via (at 141.2395 79.7229) (size 0.8) (drill 0.4) (layers "F.Cu" "B.Cu") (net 16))
 (segment (start 144.9562 91.0428) (end 141.0378 91.0428) (width 0.3) (layer "B.Cu") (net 16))
 (segment (start 141.0378 91.0428) (end 139.535 89.54) (width 0.3) (layer "B.Cu") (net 16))
 (segment (start 145.7657 84.2491) (end 145.7657 90.2333) (width 0.3) (layer "B.Cu") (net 16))
 (segment (start 141.2395 79.7229) (end 145.7657 84.2491) (width 0.3) (layer "B.Cu") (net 16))
 (segment (start 145.7657 90.2333) (end 144.9562 91.0428) (width 0.3) (layer "B.Cu") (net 16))
 (segment (start 148.463 77.8373) (end 147.0641 79.2362) (width 0.3) (layer "F.Cu") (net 17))
 (segment (start 148.463 77.724) (end 148.463 77.8373) (width 0.3) (layer "F.Cu") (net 17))
 (via (at 147.0641 79.2362) (size 0.8) (drill 0.4) (layers "F.Cu" "B.Cu") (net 17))
 (segment (start 145.1433 91.4947) (end 147.0641 89.5739) (width 0.3) (layer "B.Cu") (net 17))
 (segment (start 140.5645 91.4947) (end 145.1433 91.4947) (width 0.3) (layer "B.Cu") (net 17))
 (segment (start 147.0641 89.5739) (end 147.0641 79.2362) (width 0.3) (layer "B.Cu") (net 17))
 (segment (start 138.735 89.6652) (end 140.5645 91.4947) (width 0.3) (layer "B.Cu") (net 17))
 (segment (start 138.735 89.54) (end 138.735 89.6652) (width 0.3) (layer "B.Cu") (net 17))
 (segment (start 144.399 77.724) (end 142.3264 79.7966) (width 0.3) (layer "F.Cu") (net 18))
 (segment (start 142.3264 79.7966) (end 142.3264 82.7476) (width 0.3) (layer "F.Cu") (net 18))
 (segment (start 142.3264 82.7476) (end 141.8889 83.1851) (width 0.3) (layer "F.Cu") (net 18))
 (via (at 141.8889 83.1851) (size 0.8) (drill 0.4) (layers "F.Cu" "B.Cu") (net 18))
 (segment (start 138.4944 86.5796) (end 141.8889 83.1851) (width 0.3) (layer "B.Cu") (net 18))
 (segment (start 138.4944 88.8307) (end 138.4944 86.5796) (width 0.3) (layer "B.Cu") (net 18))
 (segment (start 137.935 89.3901) (end 138.4944 88.8307) (width 0.3) (layer "B.Cu") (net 18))
 (segment (start 137.935 89.54) (end 137.935 89.3901) (width 0.3) (layer "B.Cu") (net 18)))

